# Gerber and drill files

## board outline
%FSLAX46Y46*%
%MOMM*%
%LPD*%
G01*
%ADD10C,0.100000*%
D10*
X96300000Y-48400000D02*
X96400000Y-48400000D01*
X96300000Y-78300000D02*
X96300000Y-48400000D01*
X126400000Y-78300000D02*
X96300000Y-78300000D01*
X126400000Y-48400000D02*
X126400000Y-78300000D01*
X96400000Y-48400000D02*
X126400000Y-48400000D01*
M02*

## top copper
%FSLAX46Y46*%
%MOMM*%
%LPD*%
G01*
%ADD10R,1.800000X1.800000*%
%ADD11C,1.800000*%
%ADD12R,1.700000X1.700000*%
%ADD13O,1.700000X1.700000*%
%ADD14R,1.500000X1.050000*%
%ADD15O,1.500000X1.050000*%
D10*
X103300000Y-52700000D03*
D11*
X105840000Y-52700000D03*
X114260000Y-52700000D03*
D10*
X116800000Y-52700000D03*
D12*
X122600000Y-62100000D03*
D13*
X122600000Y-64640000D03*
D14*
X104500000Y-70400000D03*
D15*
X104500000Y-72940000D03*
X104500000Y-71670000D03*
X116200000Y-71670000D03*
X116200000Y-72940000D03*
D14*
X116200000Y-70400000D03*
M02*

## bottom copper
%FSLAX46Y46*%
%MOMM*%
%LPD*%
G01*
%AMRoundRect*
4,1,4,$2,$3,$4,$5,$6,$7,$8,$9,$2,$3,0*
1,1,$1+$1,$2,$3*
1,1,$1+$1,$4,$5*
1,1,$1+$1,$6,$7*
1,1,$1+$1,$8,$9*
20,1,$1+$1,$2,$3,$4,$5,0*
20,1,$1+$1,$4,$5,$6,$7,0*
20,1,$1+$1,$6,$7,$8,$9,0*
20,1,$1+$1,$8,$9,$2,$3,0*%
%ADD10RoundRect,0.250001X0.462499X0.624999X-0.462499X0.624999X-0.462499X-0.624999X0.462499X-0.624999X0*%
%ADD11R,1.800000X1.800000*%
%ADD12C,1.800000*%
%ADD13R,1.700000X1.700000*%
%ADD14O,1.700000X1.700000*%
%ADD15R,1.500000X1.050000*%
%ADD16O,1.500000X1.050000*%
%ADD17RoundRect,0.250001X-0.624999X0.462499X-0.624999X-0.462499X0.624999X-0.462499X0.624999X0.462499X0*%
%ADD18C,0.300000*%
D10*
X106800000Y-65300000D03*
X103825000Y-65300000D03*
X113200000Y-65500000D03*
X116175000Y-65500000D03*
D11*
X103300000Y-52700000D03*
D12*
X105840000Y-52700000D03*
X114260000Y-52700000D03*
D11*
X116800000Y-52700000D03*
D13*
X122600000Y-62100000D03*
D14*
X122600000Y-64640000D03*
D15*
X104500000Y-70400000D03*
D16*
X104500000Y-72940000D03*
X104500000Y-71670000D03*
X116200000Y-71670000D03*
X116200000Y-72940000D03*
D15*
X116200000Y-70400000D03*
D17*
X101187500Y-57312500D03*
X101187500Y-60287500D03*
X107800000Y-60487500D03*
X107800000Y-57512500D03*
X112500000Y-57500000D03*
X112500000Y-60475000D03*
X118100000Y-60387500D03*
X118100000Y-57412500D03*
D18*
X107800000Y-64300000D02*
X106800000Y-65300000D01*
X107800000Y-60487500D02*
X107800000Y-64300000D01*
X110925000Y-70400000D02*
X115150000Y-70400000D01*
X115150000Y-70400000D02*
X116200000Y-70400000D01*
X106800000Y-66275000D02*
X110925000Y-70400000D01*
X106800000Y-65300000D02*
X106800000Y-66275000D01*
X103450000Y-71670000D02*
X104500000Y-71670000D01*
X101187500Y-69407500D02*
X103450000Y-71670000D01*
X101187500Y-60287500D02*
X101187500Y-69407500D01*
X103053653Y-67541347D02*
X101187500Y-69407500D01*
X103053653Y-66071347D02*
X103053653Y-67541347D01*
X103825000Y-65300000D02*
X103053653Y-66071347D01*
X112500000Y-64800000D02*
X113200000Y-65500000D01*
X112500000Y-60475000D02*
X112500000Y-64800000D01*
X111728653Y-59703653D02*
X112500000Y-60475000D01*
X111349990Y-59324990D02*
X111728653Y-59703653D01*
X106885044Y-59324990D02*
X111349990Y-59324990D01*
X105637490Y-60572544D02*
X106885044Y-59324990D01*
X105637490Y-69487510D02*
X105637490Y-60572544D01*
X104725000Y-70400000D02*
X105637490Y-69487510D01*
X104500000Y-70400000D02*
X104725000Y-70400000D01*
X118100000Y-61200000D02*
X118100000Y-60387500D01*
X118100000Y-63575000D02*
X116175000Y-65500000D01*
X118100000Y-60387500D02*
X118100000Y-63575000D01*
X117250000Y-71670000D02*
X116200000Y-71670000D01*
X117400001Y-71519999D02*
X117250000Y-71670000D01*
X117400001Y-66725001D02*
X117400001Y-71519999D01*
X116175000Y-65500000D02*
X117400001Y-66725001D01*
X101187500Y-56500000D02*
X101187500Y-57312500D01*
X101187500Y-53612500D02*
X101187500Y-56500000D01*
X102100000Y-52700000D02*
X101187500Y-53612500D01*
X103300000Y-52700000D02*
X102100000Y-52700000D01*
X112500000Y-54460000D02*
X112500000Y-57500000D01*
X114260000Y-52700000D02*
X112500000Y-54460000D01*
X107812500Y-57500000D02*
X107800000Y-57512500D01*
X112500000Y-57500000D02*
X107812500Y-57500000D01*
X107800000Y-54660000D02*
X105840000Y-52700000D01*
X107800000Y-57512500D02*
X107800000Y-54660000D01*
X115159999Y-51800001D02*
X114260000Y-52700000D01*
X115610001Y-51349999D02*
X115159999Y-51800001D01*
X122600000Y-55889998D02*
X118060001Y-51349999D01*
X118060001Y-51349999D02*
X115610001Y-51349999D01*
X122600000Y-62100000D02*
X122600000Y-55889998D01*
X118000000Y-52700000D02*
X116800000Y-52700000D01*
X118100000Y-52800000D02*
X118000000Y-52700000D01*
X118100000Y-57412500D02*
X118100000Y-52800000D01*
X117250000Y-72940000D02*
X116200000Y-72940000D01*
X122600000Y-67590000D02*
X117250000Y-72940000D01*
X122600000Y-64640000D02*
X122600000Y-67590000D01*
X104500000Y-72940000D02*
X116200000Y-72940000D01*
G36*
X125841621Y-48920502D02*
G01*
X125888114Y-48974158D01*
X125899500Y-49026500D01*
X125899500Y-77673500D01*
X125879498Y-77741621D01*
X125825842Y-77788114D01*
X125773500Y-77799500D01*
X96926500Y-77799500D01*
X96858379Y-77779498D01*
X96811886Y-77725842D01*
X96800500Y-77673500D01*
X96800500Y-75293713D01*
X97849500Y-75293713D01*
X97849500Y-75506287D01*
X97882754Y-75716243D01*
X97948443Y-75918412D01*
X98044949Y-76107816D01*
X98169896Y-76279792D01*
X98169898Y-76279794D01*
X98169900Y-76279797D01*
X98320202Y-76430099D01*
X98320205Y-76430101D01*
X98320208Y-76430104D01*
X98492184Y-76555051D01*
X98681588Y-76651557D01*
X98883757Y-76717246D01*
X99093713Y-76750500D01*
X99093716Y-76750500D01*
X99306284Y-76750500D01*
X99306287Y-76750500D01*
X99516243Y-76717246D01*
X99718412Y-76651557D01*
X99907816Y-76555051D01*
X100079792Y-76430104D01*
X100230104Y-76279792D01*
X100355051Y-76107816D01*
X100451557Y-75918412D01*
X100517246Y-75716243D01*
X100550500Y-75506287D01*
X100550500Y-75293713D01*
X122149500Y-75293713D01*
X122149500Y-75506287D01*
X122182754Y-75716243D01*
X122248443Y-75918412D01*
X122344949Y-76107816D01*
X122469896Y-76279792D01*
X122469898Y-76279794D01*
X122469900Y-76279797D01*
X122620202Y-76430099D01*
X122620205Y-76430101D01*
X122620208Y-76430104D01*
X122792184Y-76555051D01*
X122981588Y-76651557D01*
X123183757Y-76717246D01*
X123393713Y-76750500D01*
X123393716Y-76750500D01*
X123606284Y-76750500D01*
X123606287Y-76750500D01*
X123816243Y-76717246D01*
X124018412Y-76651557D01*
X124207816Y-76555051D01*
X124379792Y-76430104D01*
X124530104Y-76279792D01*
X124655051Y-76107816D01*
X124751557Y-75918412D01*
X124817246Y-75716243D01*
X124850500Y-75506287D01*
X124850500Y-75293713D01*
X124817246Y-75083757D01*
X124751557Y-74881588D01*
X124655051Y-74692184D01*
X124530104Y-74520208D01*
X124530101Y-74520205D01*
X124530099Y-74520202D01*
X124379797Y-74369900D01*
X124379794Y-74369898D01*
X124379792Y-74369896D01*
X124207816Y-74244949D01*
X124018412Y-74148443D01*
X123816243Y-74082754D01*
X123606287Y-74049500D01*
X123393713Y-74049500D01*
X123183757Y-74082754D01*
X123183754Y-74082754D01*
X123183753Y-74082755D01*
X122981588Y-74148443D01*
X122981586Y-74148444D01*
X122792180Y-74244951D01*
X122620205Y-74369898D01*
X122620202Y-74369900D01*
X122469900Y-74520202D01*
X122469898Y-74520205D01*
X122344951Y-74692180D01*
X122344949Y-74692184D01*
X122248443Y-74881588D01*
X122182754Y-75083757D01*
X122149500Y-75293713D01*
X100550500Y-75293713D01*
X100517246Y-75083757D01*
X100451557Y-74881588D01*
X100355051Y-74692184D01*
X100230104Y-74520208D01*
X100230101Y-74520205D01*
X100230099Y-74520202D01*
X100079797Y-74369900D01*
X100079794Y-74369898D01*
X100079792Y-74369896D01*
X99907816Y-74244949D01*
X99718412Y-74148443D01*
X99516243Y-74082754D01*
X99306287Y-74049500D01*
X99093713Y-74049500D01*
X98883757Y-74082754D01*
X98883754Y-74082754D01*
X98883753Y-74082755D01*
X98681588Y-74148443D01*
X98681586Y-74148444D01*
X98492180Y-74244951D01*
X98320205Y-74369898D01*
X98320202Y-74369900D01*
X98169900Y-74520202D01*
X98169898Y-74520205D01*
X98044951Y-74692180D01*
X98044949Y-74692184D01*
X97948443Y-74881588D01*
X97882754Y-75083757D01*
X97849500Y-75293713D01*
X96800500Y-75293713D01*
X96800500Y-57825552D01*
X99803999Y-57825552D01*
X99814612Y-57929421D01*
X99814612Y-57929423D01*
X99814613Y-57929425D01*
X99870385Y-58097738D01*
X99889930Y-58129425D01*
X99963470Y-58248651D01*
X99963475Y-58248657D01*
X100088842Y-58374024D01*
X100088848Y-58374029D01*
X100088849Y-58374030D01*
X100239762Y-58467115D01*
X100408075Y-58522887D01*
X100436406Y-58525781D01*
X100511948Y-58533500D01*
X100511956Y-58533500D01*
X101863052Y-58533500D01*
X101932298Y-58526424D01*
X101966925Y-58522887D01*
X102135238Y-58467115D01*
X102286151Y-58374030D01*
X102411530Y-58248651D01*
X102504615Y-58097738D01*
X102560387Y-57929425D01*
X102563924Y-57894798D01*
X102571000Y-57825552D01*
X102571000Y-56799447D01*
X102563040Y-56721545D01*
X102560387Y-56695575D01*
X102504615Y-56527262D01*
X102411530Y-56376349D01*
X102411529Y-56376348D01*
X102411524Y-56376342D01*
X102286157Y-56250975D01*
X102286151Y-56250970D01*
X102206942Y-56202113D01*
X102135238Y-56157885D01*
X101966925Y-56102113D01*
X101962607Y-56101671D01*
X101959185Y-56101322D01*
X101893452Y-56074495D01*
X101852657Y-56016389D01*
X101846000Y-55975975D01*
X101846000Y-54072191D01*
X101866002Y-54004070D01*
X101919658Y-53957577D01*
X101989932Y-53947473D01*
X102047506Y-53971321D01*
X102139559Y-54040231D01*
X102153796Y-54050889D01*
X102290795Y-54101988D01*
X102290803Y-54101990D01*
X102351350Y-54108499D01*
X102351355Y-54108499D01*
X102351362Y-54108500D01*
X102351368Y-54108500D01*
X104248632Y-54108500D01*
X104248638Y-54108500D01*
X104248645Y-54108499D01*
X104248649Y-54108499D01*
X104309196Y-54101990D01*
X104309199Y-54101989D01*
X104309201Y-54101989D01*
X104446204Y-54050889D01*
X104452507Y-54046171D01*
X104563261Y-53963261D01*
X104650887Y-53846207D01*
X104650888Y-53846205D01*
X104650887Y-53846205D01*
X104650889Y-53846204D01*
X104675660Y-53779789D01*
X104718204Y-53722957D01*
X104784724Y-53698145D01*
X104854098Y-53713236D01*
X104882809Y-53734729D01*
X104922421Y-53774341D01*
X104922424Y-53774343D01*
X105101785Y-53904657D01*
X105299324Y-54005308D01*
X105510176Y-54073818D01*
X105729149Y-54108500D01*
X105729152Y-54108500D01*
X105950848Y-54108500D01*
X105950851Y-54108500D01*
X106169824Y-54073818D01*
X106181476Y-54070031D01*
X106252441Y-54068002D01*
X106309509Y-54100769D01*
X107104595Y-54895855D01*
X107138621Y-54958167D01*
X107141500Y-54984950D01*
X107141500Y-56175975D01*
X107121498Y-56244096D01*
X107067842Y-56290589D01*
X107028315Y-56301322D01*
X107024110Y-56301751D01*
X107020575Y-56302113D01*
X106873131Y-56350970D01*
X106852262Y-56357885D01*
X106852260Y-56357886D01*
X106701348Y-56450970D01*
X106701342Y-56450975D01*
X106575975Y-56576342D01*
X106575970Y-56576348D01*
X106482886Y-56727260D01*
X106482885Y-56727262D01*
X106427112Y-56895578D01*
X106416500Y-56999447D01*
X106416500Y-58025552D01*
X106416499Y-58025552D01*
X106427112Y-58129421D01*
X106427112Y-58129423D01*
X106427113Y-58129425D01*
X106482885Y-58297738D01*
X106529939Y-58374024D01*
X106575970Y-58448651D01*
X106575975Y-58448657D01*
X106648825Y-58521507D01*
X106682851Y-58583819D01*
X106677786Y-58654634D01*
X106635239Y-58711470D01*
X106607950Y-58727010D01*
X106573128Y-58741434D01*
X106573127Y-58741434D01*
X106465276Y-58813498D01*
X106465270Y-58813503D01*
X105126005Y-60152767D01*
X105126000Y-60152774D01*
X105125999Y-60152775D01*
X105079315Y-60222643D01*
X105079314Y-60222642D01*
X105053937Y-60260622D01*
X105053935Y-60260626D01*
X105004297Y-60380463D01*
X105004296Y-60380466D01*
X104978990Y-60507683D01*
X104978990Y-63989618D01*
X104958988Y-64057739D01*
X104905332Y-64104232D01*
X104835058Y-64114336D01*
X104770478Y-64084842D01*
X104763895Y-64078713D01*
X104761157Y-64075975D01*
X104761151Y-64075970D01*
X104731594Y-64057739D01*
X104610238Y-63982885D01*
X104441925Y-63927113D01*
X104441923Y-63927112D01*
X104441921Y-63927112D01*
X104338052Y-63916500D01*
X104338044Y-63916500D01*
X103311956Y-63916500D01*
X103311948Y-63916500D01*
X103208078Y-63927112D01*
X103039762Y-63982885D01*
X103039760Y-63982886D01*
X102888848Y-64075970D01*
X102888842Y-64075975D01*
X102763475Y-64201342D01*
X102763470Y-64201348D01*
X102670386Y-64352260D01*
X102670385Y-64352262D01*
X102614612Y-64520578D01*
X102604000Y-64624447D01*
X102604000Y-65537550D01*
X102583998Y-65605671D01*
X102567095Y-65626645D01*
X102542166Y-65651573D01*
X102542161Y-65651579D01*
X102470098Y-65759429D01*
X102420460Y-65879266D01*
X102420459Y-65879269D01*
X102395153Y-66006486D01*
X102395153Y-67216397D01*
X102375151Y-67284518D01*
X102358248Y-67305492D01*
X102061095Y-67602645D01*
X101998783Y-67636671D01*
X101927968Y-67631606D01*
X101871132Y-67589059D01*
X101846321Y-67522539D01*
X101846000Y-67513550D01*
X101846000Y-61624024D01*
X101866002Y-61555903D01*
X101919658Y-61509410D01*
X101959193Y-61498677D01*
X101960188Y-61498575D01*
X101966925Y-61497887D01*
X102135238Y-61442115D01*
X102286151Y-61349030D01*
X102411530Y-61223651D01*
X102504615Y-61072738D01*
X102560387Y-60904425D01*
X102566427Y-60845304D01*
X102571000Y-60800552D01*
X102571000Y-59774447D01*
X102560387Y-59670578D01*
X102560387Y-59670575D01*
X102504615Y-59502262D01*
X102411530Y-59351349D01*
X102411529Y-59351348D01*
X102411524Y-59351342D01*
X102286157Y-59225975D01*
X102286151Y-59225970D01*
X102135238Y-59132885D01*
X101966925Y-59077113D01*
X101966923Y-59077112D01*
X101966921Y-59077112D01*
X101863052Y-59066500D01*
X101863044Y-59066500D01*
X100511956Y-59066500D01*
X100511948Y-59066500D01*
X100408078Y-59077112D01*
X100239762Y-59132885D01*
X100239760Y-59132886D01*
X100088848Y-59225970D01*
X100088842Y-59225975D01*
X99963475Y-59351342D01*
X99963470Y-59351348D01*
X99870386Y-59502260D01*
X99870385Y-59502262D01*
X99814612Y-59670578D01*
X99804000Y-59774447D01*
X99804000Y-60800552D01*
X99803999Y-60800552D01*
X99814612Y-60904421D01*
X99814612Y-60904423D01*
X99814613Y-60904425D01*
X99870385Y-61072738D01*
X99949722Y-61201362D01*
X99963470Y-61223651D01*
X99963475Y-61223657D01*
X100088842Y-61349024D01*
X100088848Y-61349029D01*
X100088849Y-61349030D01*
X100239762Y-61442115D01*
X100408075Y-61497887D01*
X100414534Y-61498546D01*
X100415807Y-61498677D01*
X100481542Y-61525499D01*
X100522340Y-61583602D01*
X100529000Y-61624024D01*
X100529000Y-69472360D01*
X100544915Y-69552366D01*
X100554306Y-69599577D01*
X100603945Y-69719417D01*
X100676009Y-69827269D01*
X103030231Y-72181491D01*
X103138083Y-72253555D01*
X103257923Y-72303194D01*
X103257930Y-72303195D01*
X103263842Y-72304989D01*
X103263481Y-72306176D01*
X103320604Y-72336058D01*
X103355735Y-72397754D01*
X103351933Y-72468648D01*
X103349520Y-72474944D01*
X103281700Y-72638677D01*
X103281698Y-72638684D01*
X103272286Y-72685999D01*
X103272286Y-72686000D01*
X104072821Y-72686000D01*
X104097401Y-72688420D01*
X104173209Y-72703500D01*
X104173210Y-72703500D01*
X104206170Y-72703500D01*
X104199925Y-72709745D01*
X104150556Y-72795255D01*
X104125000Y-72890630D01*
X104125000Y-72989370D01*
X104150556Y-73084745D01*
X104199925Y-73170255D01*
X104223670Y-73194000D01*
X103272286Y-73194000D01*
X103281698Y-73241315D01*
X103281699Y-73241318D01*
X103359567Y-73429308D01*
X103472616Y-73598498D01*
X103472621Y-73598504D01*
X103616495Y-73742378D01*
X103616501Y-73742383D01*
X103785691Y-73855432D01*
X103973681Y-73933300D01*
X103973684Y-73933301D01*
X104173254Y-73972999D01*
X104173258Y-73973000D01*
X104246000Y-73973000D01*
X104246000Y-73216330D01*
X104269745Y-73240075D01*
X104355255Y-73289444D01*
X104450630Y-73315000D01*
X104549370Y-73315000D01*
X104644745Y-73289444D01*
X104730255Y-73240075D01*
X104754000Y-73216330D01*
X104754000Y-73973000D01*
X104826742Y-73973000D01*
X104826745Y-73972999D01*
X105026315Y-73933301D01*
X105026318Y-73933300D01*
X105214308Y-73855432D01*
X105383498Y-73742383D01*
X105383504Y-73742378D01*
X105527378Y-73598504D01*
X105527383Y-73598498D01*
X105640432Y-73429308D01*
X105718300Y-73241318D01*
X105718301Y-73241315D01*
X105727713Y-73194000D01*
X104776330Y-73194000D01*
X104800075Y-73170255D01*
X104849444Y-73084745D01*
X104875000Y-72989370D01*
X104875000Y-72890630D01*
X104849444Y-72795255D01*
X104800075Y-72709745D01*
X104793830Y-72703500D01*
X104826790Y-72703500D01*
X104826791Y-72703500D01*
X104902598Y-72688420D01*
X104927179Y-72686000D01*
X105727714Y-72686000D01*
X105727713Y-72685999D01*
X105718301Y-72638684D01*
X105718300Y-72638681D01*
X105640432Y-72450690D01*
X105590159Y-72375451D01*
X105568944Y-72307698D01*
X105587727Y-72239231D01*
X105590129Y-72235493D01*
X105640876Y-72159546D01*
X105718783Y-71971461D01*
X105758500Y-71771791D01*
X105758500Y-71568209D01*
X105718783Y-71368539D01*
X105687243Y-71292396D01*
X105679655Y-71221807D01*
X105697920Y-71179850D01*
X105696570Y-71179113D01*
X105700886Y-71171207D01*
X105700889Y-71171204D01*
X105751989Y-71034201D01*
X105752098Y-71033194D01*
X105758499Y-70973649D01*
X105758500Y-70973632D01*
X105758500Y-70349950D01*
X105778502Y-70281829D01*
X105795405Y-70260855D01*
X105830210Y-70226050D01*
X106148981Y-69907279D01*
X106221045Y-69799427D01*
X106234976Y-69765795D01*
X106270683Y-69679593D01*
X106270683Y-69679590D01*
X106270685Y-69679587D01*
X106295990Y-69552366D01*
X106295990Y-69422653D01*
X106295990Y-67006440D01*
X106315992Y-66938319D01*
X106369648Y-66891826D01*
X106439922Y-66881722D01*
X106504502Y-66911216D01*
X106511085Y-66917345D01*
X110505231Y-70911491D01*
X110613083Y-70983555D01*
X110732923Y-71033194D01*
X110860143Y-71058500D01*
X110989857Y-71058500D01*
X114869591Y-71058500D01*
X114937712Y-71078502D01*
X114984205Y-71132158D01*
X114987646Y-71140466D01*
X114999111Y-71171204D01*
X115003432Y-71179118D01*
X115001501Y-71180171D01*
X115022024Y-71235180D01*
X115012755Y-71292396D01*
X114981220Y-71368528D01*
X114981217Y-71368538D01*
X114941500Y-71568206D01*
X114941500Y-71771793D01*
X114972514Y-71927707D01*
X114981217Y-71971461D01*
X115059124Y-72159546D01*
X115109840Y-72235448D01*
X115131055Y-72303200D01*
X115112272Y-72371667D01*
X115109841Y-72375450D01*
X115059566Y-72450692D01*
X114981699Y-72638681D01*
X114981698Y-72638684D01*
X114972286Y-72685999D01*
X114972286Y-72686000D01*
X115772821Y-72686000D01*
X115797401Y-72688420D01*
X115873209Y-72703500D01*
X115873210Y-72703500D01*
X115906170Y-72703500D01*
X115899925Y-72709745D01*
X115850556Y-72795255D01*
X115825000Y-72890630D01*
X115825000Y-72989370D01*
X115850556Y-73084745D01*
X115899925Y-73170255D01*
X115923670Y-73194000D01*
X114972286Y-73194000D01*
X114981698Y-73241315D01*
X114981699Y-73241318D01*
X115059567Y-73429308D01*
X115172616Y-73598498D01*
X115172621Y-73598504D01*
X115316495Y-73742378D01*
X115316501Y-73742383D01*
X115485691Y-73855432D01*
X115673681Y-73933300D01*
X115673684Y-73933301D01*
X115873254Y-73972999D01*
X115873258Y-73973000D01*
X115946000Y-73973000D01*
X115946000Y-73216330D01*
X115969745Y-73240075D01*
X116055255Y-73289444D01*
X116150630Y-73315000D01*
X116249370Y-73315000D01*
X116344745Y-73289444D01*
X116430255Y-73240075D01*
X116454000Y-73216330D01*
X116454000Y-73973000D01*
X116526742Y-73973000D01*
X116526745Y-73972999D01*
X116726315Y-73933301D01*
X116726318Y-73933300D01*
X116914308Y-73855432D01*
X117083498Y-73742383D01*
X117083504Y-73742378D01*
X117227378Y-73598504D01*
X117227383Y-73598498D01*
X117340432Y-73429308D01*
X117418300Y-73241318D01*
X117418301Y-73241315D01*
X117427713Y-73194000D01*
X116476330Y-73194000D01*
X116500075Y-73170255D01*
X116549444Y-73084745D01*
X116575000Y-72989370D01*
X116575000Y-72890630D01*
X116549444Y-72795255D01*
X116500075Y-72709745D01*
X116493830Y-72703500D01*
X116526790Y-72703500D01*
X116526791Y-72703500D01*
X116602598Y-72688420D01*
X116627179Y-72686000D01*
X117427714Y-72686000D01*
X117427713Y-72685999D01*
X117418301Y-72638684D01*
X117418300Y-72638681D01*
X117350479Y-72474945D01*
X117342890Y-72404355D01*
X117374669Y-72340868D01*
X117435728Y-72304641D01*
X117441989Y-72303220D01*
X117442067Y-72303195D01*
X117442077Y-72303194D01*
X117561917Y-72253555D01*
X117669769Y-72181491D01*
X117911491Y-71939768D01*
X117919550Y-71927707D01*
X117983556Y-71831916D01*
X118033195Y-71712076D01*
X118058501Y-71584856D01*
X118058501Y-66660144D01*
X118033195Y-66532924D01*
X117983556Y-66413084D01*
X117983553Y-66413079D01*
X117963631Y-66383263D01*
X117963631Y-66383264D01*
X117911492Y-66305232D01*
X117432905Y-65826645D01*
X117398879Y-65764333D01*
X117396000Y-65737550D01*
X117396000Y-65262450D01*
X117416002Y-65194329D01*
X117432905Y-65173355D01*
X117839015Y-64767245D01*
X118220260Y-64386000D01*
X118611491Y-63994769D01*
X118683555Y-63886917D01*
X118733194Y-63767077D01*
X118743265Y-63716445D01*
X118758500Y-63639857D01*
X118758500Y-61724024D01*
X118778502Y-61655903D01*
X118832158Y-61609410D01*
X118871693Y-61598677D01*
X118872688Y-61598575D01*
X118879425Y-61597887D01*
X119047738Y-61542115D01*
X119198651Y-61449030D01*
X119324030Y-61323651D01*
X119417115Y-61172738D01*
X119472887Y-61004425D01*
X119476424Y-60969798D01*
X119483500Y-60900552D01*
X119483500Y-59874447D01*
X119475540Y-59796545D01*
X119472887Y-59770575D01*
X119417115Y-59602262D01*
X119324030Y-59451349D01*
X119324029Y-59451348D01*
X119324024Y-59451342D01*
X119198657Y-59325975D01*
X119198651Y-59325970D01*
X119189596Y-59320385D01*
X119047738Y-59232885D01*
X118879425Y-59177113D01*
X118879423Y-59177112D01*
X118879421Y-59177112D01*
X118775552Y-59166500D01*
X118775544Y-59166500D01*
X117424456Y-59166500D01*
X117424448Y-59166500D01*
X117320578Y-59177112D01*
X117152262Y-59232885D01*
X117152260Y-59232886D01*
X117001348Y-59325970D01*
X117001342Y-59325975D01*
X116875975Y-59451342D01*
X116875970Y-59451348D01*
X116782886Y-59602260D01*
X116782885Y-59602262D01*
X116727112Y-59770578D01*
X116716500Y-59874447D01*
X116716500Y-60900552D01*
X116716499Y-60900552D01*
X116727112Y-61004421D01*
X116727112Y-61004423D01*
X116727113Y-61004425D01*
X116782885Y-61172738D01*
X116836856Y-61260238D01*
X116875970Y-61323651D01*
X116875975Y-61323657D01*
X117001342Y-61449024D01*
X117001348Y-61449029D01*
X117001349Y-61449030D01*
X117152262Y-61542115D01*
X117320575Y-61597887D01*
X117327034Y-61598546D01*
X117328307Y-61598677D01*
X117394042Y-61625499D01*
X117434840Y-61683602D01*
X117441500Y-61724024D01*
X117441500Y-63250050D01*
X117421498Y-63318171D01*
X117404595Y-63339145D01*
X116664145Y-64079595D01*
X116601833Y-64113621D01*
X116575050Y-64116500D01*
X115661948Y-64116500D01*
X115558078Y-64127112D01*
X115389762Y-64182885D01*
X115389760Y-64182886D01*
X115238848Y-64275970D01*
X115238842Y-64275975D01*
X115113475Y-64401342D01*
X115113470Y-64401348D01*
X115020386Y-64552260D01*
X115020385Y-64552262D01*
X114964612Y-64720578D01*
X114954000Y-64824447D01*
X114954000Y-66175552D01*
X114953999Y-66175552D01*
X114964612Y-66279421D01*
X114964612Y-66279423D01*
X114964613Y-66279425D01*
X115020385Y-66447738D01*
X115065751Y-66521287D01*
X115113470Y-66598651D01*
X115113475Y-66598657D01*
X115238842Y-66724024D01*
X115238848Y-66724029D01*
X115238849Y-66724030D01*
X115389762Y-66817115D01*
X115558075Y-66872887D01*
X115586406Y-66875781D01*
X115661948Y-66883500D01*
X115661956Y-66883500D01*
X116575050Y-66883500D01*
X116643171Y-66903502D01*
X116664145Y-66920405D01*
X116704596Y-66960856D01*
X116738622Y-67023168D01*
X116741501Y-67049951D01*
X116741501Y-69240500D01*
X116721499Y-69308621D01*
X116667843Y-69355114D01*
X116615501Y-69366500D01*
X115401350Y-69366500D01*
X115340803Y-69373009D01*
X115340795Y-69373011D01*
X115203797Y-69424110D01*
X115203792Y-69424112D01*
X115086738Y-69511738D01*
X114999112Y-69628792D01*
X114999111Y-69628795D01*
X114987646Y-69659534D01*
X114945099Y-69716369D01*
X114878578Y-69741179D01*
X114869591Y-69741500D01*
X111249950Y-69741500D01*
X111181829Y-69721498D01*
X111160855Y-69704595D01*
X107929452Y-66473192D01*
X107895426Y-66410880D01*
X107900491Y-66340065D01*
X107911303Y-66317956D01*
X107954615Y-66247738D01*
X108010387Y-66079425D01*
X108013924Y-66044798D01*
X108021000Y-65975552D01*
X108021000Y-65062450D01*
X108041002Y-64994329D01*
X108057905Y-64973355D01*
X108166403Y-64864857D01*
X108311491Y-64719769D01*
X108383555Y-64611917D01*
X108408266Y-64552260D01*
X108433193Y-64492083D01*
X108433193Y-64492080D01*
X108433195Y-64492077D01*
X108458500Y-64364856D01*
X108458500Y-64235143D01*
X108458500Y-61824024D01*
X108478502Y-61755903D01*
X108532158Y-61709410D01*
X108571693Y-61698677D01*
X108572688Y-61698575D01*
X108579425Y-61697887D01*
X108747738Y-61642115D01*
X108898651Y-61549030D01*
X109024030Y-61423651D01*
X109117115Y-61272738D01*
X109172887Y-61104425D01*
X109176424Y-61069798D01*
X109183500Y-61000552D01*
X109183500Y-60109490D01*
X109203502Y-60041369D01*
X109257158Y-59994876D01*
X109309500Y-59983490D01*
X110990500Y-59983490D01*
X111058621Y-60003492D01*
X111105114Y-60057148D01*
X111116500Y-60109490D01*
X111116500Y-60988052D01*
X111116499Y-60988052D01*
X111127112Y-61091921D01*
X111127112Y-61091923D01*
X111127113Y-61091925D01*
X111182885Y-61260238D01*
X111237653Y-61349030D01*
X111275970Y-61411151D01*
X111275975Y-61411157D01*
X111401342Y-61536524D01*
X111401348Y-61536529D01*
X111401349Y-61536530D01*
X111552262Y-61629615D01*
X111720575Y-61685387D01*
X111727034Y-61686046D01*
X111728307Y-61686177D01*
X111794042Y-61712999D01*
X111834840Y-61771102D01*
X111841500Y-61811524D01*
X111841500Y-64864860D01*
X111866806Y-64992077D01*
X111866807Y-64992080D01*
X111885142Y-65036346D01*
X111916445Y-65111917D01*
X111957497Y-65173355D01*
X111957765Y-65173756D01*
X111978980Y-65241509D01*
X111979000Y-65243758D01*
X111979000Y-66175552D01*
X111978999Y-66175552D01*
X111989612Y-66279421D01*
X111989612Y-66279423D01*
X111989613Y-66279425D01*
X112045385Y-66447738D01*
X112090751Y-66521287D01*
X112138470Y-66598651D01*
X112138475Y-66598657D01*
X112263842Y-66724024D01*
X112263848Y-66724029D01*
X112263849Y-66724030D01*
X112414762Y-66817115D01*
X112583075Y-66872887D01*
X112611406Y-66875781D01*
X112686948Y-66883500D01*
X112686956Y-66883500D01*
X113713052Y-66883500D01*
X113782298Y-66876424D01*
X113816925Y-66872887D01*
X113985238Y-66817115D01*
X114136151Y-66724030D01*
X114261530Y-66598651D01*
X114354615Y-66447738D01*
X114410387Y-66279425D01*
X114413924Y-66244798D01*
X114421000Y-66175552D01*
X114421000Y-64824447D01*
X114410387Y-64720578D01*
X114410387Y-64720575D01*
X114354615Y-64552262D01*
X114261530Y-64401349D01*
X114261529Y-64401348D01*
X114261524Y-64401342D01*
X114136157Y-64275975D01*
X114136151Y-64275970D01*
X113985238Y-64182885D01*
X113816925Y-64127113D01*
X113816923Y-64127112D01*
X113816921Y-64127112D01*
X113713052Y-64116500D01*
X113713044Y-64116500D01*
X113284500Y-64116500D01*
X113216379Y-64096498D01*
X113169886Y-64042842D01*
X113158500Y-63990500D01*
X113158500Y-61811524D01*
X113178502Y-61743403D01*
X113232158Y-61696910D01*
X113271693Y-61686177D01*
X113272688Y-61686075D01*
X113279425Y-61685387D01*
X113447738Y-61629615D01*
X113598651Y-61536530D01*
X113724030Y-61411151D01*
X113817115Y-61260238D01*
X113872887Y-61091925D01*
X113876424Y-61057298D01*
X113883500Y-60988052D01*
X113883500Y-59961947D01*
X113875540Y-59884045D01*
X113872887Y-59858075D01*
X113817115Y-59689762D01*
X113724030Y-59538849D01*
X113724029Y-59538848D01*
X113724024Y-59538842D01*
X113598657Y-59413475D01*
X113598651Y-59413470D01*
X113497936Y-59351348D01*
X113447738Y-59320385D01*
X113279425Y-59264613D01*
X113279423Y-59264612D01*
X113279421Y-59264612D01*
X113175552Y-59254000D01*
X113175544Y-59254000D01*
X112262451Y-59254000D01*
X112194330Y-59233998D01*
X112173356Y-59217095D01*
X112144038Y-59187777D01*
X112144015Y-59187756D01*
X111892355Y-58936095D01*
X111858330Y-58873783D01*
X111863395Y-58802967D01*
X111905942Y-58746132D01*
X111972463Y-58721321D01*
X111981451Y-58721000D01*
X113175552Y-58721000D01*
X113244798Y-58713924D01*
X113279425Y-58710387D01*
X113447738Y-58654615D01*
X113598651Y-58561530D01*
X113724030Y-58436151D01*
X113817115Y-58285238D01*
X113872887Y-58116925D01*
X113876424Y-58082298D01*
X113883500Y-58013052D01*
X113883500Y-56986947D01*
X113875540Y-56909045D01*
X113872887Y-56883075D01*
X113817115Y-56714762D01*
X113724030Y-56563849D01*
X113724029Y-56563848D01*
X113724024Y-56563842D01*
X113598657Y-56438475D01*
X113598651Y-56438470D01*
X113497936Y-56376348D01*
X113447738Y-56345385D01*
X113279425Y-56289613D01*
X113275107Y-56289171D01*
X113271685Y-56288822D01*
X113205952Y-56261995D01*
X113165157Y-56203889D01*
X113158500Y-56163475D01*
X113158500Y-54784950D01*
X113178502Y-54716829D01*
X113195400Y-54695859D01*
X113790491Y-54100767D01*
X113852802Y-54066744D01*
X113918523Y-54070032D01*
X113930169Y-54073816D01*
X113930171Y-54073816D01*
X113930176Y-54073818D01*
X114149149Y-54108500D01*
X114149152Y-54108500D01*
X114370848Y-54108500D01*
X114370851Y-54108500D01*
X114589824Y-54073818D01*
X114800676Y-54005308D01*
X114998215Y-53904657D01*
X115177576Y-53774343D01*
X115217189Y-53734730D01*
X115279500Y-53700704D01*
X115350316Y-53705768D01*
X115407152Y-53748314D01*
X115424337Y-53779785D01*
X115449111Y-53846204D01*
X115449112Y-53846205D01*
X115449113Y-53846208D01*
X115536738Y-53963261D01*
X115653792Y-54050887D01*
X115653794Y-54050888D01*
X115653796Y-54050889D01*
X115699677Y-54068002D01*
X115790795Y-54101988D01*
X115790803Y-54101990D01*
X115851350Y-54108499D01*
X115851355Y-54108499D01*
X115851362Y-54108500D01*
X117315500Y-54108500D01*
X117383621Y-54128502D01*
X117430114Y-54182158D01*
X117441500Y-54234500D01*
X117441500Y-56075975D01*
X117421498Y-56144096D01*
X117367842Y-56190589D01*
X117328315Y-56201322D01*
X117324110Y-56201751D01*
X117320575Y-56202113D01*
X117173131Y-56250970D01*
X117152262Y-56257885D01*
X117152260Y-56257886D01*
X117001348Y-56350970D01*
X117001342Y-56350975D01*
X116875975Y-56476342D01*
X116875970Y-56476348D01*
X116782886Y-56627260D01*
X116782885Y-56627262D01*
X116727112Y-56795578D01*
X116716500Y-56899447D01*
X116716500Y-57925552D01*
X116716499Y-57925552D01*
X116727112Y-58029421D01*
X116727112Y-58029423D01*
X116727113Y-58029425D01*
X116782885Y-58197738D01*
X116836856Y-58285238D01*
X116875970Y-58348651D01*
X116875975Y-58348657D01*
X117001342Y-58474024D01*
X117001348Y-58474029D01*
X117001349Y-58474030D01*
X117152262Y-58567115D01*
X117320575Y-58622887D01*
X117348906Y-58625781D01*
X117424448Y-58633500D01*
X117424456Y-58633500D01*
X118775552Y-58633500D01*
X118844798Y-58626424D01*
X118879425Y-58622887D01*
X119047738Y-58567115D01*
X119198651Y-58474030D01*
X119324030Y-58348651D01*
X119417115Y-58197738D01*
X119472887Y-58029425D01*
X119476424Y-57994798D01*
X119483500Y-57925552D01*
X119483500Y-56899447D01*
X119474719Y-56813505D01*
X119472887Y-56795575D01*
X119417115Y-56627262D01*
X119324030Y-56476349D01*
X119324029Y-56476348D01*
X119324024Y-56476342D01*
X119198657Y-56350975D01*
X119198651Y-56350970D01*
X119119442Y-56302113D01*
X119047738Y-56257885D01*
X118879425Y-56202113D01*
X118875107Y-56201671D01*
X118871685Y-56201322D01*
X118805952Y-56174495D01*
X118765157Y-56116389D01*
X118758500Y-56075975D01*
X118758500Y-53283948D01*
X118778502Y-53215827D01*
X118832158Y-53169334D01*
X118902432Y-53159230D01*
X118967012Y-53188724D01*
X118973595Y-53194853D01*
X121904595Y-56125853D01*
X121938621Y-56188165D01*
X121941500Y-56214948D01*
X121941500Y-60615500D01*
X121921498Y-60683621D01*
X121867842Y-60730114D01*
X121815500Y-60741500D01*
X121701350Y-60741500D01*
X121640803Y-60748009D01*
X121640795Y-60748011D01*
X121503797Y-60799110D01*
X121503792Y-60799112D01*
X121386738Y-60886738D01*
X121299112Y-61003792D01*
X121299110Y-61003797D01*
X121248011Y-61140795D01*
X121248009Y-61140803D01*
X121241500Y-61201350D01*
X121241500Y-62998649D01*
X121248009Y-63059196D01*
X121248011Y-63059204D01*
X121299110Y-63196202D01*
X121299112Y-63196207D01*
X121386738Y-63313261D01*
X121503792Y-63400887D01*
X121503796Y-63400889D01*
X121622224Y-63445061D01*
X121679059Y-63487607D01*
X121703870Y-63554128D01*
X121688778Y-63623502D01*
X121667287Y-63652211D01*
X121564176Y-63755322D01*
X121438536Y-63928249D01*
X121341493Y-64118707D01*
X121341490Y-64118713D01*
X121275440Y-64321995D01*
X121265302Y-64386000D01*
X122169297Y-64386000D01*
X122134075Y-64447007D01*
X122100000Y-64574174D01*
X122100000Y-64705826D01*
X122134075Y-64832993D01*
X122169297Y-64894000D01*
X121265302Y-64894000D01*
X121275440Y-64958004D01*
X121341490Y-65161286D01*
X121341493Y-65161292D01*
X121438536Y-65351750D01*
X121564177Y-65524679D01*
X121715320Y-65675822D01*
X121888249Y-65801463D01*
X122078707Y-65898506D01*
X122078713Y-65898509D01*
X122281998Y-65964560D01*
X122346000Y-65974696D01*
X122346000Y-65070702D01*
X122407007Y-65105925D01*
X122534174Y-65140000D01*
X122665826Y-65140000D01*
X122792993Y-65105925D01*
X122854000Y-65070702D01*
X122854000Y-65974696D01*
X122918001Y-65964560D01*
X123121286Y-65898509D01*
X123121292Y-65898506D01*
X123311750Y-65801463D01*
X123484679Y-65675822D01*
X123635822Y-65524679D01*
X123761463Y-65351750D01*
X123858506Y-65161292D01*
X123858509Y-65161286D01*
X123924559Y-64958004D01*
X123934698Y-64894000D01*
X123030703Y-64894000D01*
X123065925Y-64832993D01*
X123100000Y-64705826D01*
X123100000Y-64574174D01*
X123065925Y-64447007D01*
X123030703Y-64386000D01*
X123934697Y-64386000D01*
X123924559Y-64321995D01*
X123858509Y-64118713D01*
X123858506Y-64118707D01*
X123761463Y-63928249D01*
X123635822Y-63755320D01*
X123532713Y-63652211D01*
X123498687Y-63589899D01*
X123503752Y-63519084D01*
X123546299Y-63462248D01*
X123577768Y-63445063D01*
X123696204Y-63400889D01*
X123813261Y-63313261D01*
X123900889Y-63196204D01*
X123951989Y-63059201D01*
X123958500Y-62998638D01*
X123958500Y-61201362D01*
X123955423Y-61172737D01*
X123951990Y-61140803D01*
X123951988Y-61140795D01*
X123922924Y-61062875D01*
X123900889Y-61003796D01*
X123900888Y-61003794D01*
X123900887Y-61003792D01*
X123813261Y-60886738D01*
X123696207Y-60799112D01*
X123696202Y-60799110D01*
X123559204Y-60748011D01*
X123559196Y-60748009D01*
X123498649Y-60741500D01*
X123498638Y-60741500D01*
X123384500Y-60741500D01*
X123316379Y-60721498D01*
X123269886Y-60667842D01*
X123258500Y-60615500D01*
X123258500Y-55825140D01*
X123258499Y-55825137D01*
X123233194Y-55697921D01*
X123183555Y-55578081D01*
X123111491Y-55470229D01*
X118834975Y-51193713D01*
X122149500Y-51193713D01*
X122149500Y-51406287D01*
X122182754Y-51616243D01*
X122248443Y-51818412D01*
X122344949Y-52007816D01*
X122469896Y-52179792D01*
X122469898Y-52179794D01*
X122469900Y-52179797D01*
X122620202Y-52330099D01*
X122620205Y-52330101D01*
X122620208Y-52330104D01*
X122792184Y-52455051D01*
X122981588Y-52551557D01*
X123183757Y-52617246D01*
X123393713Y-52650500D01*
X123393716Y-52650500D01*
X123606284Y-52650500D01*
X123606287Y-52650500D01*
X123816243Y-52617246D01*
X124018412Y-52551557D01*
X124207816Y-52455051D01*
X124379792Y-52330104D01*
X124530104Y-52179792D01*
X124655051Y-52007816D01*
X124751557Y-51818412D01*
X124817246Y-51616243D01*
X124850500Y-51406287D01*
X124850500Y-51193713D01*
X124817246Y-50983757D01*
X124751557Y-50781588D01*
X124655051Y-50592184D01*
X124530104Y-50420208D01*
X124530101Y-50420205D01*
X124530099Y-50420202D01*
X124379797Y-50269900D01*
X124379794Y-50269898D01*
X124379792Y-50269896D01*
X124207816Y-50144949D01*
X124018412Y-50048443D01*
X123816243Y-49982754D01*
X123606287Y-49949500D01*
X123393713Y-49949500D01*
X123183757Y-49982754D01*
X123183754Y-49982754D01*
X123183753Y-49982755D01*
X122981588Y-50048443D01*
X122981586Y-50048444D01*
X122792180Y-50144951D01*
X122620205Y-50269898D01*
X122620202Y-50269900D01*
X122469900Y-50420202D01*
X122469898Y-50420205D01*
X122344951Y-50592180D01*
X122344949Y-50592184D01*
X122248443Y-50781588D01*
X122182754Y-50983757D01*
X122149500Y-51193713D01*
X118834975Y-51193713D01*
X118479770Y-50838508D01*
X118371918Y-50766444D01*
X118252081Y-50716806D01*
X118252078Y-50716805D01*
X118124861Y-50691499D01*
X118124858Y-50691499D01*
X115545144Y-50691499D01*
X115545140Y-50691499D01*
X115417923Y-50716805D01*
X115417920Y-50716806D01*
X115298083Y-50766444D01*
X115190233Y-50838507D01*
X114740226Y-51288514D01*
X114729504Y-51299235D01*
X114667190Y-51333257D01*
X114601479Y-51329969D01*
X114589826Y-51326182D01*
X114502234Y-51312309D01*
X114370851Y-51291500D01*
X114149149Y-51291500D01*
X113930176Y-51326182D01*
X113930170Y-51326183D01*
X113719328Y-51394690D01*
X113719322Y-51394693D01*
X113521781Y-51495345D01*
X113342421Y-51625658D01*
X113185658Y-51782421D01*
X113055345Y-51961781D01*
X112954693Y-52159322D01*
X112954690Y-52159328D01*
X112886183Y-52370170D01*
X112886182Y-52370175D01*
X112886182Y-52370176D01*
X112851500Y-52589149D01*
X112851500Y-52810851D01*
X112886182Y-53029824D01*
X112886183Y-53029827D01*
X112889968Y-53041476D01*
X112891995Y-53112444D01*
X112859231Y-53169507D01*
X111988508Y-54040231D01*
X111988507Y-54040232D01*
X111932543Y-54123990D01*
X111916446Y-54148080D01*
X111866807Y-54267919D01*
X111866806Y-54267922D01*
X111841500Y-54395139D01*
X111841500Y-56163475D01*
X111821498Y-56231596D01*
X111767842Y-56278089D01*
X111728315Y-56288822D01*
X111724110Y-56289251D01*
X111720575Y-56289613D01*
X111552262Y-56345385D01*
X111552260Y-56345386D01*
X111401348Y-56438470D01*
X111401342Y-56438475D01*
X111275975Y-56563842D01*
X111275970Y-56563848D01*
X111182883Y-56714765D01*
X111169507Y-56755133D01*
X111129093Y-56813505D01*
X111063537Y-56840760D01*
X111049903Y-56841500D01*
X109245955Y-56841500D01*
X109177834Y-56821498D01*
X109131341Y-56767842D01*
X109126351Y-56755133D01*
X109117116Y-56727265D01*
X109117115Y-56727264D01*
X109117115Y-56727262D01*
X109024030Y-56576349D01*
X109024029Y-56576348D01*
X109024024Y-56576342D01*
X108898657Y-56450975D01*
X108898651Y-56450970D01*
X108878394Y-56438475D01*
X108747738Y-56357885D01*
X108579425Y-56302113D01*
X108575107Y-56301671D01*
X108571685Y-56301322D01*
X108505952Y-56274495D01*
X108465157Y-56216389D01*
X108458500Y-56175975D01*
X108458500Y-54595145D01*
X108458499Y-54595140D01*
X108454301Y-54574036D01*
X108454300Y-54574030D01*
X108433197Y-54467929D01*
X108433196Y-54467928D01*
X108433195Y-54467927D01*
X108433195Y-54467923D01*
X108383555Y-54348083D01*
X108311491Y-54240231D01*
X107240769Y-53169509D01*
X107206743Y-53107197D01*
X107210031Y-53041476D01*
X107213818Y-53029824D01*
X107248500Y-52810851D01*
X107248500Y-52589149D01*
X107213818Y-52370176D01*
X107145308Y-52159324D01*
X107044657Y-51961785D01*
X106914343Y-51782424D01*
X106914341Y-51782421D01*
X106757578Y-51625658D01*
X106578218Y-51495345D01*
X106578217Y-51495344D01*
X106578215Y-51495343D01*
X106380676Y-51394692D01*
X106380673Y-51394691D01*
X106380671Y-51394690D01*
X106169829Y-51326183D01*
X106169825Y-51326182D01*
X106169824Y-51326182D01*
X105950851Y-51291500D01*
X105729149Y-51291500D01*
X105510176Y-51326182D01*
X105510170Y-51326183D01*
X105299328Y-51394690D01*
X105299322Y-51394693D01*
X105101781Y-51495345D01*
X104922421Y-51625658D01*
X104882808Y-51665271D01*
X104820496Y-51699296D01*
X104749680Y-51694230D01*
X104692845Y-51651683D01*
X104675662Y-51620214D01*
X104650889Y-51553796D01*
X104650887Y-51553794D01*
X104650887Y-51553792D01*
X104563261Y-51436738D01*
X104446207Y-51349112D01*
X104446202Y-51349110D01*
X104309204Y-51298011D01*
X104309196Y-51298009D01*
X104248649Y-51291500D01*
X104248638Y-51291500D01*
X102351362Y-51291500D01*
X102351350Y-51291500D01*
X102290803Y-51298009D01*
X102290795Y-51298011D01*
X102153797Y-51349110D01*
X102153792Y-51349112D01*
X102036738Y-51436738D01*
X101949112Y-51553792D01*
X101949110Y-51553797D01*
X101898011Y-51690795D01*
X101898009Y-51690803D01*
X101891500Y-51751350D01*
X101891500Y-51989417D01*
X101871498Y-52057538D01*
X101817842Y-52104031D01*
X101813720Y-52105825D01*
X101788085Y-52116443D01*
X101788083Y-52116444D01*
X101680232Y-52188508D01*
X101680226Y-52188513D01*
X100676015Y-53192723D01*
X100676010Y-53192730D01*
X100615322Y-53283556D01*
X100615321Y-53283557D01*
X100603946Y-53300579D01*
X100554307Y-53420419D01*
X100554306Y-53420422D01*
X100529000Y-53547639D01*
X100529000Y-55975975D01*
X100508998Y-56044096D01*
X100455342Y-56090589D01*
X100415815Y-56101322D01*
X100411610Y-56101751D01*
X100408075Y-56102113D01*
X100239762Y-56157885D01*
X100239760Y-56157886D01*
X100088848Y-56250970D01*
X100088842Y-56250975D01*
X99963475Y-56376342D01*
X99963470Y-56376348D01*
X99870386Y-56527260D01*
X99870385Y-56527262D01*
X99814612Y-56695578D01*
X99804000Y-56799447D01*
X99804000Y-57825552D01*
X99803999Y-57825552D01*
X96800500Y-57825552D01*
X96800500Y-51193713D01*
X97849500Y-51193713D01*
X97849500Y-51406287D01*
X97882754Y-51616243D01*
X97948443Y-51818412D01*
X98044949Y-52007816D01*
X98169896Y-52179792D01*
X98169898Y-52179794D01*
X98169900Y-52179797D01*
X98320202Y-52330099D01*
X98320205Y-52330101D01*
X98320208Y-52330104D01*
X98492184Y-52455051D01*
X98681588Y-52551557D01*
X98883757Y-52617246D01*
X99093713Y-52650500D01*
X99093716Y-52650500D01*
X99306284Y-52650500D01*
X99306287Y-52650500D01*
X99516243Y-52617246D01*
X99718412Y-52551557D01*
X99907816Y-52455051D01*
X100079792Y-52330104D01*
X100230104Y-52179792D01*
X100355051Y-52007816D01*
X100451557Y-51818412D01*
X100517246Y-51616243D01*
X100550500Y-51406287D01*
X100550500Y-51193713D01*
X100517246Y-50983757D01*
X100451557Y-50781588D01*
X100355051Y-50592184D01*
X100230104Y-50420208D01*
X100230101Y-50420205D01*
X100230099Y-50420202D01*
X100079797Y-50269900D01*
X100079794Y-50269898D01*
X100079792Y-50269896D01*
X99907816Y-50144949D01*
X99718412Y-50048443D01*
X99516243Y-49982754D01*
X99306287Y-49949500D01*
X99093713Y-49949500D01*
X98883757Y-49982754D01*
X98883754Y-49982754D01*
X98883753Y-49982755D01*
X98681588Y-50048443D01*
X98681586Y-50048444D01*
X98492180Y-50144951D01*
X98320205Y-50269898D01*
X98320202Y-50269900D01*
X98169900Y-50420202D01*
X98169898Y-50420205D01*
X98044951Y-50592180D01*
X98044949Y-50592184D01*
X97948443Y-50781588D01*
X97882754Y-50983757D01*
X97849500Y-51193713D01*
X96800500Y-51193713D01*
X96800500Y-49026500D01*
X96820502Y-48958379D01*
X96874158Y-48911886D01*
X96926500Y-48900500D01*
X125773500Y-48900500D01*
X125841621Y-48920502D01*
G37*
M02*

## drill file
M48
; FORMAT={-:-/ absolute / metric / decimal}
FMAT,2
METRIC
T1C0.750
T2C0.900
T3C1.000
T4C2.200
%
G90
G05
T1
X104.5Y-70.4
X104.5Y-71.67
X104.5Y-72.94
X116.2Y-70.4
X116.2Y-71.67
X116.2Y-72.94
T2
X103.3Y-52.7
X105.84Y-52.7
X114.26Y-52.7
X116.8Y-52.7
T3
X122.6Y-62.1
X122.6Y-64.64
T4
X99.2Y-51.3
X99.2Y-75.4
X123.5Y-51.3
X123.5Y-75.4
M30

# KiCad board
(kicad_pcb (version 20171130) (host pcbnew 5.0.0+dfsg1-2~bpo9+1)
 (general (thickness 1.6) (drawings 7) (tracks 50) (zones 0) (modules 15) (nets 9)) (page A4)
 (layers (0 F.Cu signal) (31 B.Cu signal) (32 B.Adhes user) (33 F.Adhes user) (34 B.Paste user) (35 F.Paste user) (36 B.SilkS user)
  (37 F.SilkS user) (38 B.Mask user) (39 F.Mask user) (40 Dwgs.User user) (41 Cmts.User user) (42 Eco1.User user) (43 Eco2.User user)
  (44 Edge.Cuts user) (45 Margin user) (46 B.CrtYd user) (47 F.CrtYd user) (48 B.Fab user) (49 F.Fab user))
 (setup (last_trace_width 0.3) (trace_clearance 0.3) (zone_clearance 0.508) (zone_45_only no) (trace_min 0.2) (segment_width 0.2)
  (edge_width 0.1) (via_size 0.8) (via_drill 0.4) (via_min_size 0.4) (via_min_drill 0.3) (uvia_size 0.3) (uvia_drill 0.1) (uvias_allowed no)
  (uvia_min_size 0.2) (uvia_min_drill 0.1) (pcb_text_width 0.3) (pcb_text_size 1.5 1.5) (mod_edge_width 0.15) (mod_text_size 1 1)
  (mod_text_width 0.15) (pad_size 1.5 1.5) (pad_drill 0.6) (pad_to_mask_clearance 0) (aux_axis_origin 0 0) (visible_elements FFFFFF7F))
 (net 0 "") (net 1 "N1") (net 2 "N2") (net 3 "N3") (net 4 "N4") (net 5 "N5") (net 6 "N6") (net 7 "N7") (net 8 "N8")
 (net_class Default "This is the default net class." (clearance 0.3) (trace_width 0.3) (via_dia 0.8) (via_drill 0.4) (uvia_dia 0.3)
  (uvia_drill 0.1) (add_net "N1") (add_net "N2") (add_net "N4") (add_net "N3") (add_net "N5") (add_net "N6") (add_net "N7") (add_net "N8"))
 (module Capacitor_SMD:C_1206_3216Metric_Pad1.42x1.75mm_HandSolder (layer B.Cu) (at 105.3125 65.3 180)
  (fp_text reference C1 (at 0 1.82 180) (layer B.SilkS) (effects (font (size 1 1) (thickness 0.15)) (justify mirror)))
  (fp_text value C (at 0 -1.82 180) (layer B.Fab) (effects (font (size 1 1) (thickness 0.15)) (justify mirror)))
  (pad 1 smd roundrect (at -1.4875 0 180) (size 1.425 1.75) (layers B.Cu B.Paste B.Mask) (roundrect_rratio 0.175439) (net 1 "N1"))
  (pad 2 smd roundrect (at 1.4875 0 180) (size 1.425 1.75) (layers B.Cu B.Paste B.Mask) (roundrect_rratio 0.175439) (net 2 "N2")))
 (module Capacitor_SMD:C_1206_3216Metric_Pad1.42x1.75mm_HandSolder (layer B.Cu) (at 114.6875 65.5 180)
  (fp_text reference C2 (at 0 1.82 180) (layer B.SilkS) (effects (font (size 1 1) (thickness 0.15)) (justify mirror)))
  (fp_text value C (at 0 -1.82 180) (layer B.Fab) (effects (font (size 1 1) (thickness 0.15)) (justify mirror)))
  (pad 2 smd roundrect (at 1.4875 0 180) (size 1.425 1.75) (layers B.Cu B.Paste B.Mask) (roundrect_rratio 0.175439) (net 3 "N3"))
  (pad 1 smd roundrect (at -1.4875 0 180) (size 1.425 1.75) (layers B.Cu B.Paste B.Mask) (roundrect_rratio 0.175439) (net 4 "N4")))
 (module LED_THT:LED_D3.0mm (layer F.Cu) (at 103.3 52.7)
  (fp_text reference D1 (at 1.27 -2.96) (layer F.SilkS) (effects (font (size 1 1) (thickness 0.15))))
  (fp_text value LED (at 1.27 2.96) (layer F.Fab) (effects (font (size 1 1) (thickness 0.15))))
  (pad 1 thru_hole rect (at 0 0) (size 1.8 1.8) (drill 0.9) (layers *.Cu *.Mask) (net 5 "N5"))
  (pad 2 thru_hole circle (at 2.54 0) (size 1.8 1.8) (drill 0.9) (layers *.Cu *.Mask) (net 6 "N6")))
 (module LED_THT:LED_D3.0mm (layer F.Cu) (at 116.8 52.7 180)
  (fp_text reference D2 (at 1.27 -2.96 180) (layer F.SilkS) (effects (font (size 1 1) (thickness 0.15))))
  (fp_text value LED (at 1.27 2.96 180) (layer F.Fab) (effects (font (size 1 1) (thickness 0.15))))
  (pad 2 thru_hole circle (at 2.54 0 180) (size 1.8 1.8) (drill 0.9) (layers *.Cu *.Mask) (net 6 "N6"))
  (pad 1 thru_hole rect (at 0 0 180) (size 1.8 1.8) (drill 0.9) (layers *.Cu *.Mask) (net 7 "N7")))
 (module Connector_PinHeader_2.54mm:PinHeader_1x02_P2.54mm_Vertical (layer F.Cu) (at 122.6 62.1)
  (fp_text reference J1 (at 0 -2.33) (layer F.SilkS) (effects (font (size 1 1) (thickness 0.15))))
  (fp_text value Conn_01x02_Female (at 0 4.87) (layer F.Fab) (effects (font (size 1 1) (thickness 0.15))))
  (pad 1 thru_hole rect (at 0 0) (size 1.7 1.7) (drill 1) (layers *.Cu *.Mask) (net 6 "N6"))
  (pad 2 thru_hole oval (at 0 2.54) (size 1.7 1.7) (drill 1) (layers *.Cu *.Mask) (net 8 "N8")))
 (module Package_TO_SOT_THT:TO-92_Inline (layer F.Cu) (at 104.5 70.4 270)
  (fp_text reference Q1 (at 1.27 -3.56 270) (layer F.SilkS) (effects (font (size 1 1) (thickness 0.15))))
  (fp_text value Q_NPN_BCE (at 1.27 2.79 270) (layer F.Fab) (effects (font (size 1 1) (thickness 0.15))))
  (pad 1 thru_hole rect (at 0 0 270) (size 1.05 1.5) (drill 0.75) (layers *.Cu *.Mask) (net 3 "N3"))
  (pad 3 thru_hole oval (at 2.54 0 270) (size 1.05 1.5) (drill 0.75) (layers *.Cu *.Mask) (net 8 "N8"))
  (pad 2 thru_hole oval (at 1.27 0 270) (size 1.05 1.5) (drill 0.75) (layers *.Cu *.Mask) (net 2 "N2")))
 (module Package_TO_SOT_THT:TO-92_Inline (layer F.Cu) (at 116.2 70.4 270)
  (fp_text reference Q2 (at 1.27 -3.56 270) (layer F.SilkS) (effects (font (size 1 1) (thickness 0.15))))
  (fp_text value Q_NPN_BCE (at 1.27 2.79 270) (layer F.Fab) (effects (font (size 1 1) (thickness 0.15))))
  (pad 2 thru_hole oval (at 1.27 0 270) (size 1.05 1.5) (drill 0.75) (layers *.Cu *.Mask) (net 4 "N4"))
  (pad 3 thru_hole oval (at 2.54 0 270) (size 1.05 1.5) (drill 0.75) (layers *.Cu *.Mask) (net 8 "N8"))
  (pad 1 thru_hole rect (at 0 0 270) (size 1.05 1.5) (drill 0.75) (layers *.Cu *.Mask) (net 1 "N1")))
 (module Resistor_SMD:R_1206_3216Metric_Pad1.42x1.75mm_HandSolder (layer B.Cu) (at 101.1875 58.8 270)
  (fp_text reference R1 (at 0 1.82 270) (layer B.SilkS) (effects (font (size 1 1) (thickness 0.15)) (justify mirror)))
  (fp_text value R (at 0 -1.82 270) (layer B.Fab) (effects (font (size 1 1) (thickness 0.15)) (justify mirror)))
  (pad 1 smd roundrect (at -1.4875 0 270) (size 1.425 1.75) (layers B.Cu B.Paste B.Mask) (roundrect_rratio 0.175439) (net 5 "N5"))
  (pad 2 smd roundrect (at 1.4875 0 270) (size 1.425 1.75) (layers B.Cu B.Paste B.Mask) (roundrect_rratio 0.175439) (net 2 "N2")))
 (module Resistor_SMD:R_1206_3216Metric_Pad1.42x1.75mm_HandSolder (layer B.Cu) (at 107.8 59 270)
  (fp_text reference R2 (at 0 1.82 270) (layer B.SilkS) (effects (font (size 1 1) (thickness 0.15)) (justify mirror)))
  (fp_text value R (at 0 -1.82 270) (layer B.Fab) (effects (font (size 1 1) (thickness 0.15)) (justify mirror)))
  (pad 2 smd roundrect (at 1.4875 0 270) (size 1.425 1.75) (layers B.Cu B.Paste B.Mask) (roundrect_rratio 0.175439) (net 1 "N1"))
  (pad 1 smd roundrect (at -1.4875 0 270) (size 1.425 1.75) (layers B.Cu B.Paste B.Mask) (roundrect_rratio 0.175439) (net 6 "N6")))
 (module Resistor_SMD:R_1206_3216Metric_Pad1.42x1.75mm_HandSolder (layer B.Cu) (at 112.5 58.9875 270)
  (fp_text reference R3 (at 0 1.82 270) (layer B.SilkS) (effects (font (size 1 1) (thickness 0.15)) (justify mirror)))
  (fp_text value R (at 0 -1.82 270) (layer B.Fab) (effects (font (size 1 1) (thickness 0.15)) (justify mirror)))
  (pad 1 smd roundrect (at -1.4875 0 270) (size 1.425 1.75) (layers B.Cu B.Paste B.Mask) (roundrect_rratio 0.175439) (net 6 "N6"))
  (pad 2 smd roundrect (at 1.4875 0 270) (size 1.425 1.75) (layers B.Cu B.Paste B.Mask) (roundrect_rratio 0.175439) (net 3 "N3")))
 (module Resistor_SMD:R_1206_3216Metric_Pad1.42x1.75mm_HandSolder (layer B.Cu) (at 118.1 58.9 270)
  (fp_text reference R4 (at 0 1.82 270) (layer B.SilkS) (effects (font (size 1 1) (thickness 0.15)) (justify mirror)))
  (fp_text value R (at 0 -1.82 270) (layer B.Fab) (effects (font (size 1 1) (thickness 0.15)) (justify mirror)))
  (pad 2 smd roundrect (at 1.4875 0 270) (size 1.425 1.75) (layers B.Cu B.Paste B.Mask) (roundrect_rratio 0.175439) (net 4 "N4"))
  (pad 1 smd roundrect (at -1.4875 0 270) (size 1.425 1.75) (layers B.Cu B.Paste B.Mask) (roundrect_rratio 0.175439) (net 7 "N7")))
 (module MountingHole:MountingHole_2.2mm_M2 (layer F.Cu) (at 123.5 51.3)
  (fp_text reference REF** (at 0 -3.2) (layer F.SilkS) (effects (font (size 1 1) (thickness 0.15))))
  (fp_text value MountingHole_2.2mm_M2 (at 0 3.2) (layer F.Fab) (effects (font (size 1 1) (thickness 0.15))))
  (pad 1 np_thru_hole circle (at 0 0) (size 2.2 2.2) (drill 2.2) (layers *.Cu *.Mask)))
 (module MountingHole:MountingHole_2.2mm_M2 (layer F.Cu) (at 99.2 51.3)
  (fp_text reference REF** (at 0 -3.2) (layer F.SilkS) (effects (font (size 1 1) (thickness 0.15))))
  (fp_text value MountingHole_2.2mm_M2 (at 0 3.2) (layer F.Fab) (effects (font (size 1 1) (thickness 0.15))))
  (pad 1 np_thru_hole circle (at 0 0) (size 2.2 2.2) (drill 2.2) (layers *.Cu *.Mask)))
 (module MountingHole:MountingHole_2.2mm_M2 (layer F.Cu) (at 99.2 75.4)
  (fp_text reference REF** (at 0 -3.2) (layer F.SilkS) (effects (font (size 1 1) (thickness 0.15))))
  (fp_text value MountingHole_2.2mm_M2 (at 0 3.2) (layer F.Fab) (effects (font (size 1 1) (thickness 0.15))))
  (pad 1 np_thru_hole circle (at 0 0) (size 2.2 2.2) (drill 2.2) (layers *.Cu *.Mask)))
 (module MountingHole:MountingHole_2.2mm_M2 (layer F.Cu) (at 123.5 75.4)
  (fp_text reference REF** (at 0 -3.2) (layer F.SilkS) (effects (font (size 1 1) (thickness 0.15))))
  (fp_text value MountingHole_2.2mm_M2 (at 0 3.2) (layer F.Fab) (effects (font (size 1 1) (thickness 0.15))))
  (pad 1 np_thru_hole circle (at 0 0) (size 2.2 2.2) (drill 2.2) (layers *.Cu *.Mask)))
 (gr_line (start 96.3 48.4) (end 96.4 48.4) (layer Edge.Cuts) (width 0.1))
 (gr_line (start 96.3 78.3) (end 96.3 48.4) (layer Edge.Cuts) (width 0.1))
 (gr_line (start 126.4 78.3) (end 96.3 78.3) (layer Edge.Cuts) (width 0.1))
 (gr_line (start 126.4 48.4) (end 126.4 78.3) (layer Edge.Cuts) (width 0.1))
 (gr_line (start 96.4 48.4) (end 126.4 48.4) (layer Edge.Cuts) (width 0.1))
 (segment (start 107.8 64.3) (end 106.8 65.3) (width 0.3) (layer B.Cu) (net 1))
 (segment (start 107.8 60.4875) (end 107.8 64.3) (width 0.3) (layer B.Cu) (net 1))
 (segment (start 110.925 70.4) (end 115.15 70.4) (width 0.3) (layer B.Cu) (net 1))
 (segment (start 115.15 70.4) (end 116.2 70.4) (width 0.3) (layer B.Cu) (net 1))
 (segment (start 106.8 66.275) (end 110.925 70.4) (width 0.3) (layer B.Cu) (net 1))
 (segment (start 106.8 65.3) (end 106.8 66.275) (width 0.3) (layer B.Cu) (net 1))
 (segment (start 103.45 71.67) (end 104.5 71.67) (width 0.3) (layer B.Cu) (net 2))
 (segment (start 101.1875 69.4075) (end 103.45 71.67) (width 0.3) (layer B.Cu) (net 2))
 (segment (start 101.1875 60.2875) (end 101.1875 69.4075) (width 0.3) (layer B.Cu) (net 2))
 (segment (start 103.053653 67.541347) (end 101.1875 69.4075) (width 0.3) (layer B.Cu) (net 2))
 (segment (start 103.053653 66.071347) (end 103.053653 67.541347) (width 0.3) (layer B.Cu) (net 2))
 (segment (start 103.825 65.3) (end 103.053653 66.071347) (width 0.3) (layer B.Cu) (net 2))
 (segment (start 112.5 64.8) (end 113.2 65.5) (width 0.3) (layer B.Cu) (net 3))
 (segment (start 112.5 60.475) (end 112.5 64.8) (width 0.3) (layer B.Cu) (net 3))
 (segment (start 111.728653 59.703653) (end 112.5 60.475) (width 0.3) (layer B.Cu) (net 3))
 (segment (start 111.34999 59.32499) (end 111.728653 59.703653) (width 0.3) (layer B.Cu) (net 3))
 (segment (start 106.885044 59.32499) (end 111.34999 59.32499) (width 0.3) (layer B.Cu) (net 3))
 (segment (start 105.63749 60.572544) (end 106.885044 59.32499) (width 0.3) (layer B.Cu) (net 3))
 (segment (start 105.63749 69.48751) (end 105.63749 60.572544) (width 0.3) (layer B.Cu) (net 3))
 (segment (start 104.725 70.4) (end 105.63749 69.48751) (width 0.3) (layer B.Cu) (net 3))
 (segment (start 104.5 70.4) (end 104.725 70.4) (width 0.3) (layer B.Cu) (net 3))
 (segment (start 118.1 61.2) (end 118.1 60.3875) (width 0.3) (layer B.Cu) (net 4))
 (segment (start 118.1 63.575) (end 116.175 65.5) (width 0.3) (layer B.Cu) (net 4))
 (segment (start 118.1 60.3875) (end 118.1 63.575) (width 0.3) (layer B.Cu) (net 4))
 (segment (start 117.25 71.67) (end 116.2 71.67) (width 0.3) (layer B.Cu) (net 4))
 (segment (start 117.400001 71.519999) (end 117.25 71.67) (width 0.3) (layer B.Cu) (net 4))
 (segment (start 117.400001 66.725001) (end 117.400001 71.519999) (width 0.3) (layer B.Cu) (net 4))
 (segment (start 116.175 65.5) (end 117.400001 66.725001) (width 0.3) (layer B.Cu) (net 4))
 (segment (start 101.1875 56.5) (end 101.1875 57.3125) (width 0.3) (layer B.Cu) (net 5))
 (segment (start 101.1875 53.6125) (end 101.1875 56.5) (width 0.3) (layer B.Cu) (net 5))
 (segment (start 102.1 52.7) (end 101.1875 53.6125) (width 0.3) (layer B.Cu) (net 5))
 (segment (start 103.3 52.7) (end 102.1 52.7) (width 0.3) (layer B.Cu) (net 5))
 (segment (start 112.5 54.46) (end 112.5 57.5) (width 0.3) (layer B.Cu) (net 6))
 (segment (start 114.26 52.7) (end 112.5 54.46) (width 0.3) (layer B.Cu) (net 6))
 (segment (start 107.8125 57.5) (end 107.8 57.5125) (width 0.3) (layer B.Cu) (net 6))
 (segment (start 112.5 57.5) (end 107.8125 57.5) (width 0.3) (layer B.Cu) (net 6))
 (segment (start 107.8 54.66) (end 105.84 52.7) (width 0.3) (layer B.Cu) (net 6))
 (segment (start 107.8 57.5125) (end 107.8 54.66) (width 0.3) (layer B.Cu) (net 6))
 (segment (start 115.159999 51.800001) (end 114.26 52.7) (width 0.3) (layer B.Cu) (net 6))
 (segment (start 115.610001 51.349999) (end 115.159999 51.800001) (width 0.3) (layer B.Cu) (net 6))
 (segment (start 122.6 55.889998) (end 118.060001 51.349999) (width 0.3) (layer B.Cu) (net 6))
 (segment (start 118.060001 51.349999) (end 115.610001 51.349999) (width 0.3) (layer B.Cu) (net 6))
 (segment (start 122.6 62.1) (end 122.6 55.889998) (width 0.3) (layer B.Cu) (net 6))
 (segment (start 118 52.7) (end 116.8 52.7) (width 0.3) (layer B.Cu) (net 7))
 (segment (start 118.1 52.8) (end 118 52.7) (width 0.3) (layer B.Cu) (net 7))
 (segment (start 118.1 57.4125) (end 118.1 52.8) (width 0.3) (layer B.Cu) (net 7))
 (segment (start 117.25 72.94) (end 116.2 72.94) (width 0.3) (layer B.Cu) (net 8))
 (segment (start 122.6 67.59) (end 117.25 72.94) (width 0.3) (layer B.Cu) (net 8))
 (segment (start 122.6 64.64) (end 122.6 67.59) (width 0.3) (layer B.Cu) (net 8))
 (segment (start 104.5 72.94) (end 116.2 72.94) (width 0.3) (layer B.Cu) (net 8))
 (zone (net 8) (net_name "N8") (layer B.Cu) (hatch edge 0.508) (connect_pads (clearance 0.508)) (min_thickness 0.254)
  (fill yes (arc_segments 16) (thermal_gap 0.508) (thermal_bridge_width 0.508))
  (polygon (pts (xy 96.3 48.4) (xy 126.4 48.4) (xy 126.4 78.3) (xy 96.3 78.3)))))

